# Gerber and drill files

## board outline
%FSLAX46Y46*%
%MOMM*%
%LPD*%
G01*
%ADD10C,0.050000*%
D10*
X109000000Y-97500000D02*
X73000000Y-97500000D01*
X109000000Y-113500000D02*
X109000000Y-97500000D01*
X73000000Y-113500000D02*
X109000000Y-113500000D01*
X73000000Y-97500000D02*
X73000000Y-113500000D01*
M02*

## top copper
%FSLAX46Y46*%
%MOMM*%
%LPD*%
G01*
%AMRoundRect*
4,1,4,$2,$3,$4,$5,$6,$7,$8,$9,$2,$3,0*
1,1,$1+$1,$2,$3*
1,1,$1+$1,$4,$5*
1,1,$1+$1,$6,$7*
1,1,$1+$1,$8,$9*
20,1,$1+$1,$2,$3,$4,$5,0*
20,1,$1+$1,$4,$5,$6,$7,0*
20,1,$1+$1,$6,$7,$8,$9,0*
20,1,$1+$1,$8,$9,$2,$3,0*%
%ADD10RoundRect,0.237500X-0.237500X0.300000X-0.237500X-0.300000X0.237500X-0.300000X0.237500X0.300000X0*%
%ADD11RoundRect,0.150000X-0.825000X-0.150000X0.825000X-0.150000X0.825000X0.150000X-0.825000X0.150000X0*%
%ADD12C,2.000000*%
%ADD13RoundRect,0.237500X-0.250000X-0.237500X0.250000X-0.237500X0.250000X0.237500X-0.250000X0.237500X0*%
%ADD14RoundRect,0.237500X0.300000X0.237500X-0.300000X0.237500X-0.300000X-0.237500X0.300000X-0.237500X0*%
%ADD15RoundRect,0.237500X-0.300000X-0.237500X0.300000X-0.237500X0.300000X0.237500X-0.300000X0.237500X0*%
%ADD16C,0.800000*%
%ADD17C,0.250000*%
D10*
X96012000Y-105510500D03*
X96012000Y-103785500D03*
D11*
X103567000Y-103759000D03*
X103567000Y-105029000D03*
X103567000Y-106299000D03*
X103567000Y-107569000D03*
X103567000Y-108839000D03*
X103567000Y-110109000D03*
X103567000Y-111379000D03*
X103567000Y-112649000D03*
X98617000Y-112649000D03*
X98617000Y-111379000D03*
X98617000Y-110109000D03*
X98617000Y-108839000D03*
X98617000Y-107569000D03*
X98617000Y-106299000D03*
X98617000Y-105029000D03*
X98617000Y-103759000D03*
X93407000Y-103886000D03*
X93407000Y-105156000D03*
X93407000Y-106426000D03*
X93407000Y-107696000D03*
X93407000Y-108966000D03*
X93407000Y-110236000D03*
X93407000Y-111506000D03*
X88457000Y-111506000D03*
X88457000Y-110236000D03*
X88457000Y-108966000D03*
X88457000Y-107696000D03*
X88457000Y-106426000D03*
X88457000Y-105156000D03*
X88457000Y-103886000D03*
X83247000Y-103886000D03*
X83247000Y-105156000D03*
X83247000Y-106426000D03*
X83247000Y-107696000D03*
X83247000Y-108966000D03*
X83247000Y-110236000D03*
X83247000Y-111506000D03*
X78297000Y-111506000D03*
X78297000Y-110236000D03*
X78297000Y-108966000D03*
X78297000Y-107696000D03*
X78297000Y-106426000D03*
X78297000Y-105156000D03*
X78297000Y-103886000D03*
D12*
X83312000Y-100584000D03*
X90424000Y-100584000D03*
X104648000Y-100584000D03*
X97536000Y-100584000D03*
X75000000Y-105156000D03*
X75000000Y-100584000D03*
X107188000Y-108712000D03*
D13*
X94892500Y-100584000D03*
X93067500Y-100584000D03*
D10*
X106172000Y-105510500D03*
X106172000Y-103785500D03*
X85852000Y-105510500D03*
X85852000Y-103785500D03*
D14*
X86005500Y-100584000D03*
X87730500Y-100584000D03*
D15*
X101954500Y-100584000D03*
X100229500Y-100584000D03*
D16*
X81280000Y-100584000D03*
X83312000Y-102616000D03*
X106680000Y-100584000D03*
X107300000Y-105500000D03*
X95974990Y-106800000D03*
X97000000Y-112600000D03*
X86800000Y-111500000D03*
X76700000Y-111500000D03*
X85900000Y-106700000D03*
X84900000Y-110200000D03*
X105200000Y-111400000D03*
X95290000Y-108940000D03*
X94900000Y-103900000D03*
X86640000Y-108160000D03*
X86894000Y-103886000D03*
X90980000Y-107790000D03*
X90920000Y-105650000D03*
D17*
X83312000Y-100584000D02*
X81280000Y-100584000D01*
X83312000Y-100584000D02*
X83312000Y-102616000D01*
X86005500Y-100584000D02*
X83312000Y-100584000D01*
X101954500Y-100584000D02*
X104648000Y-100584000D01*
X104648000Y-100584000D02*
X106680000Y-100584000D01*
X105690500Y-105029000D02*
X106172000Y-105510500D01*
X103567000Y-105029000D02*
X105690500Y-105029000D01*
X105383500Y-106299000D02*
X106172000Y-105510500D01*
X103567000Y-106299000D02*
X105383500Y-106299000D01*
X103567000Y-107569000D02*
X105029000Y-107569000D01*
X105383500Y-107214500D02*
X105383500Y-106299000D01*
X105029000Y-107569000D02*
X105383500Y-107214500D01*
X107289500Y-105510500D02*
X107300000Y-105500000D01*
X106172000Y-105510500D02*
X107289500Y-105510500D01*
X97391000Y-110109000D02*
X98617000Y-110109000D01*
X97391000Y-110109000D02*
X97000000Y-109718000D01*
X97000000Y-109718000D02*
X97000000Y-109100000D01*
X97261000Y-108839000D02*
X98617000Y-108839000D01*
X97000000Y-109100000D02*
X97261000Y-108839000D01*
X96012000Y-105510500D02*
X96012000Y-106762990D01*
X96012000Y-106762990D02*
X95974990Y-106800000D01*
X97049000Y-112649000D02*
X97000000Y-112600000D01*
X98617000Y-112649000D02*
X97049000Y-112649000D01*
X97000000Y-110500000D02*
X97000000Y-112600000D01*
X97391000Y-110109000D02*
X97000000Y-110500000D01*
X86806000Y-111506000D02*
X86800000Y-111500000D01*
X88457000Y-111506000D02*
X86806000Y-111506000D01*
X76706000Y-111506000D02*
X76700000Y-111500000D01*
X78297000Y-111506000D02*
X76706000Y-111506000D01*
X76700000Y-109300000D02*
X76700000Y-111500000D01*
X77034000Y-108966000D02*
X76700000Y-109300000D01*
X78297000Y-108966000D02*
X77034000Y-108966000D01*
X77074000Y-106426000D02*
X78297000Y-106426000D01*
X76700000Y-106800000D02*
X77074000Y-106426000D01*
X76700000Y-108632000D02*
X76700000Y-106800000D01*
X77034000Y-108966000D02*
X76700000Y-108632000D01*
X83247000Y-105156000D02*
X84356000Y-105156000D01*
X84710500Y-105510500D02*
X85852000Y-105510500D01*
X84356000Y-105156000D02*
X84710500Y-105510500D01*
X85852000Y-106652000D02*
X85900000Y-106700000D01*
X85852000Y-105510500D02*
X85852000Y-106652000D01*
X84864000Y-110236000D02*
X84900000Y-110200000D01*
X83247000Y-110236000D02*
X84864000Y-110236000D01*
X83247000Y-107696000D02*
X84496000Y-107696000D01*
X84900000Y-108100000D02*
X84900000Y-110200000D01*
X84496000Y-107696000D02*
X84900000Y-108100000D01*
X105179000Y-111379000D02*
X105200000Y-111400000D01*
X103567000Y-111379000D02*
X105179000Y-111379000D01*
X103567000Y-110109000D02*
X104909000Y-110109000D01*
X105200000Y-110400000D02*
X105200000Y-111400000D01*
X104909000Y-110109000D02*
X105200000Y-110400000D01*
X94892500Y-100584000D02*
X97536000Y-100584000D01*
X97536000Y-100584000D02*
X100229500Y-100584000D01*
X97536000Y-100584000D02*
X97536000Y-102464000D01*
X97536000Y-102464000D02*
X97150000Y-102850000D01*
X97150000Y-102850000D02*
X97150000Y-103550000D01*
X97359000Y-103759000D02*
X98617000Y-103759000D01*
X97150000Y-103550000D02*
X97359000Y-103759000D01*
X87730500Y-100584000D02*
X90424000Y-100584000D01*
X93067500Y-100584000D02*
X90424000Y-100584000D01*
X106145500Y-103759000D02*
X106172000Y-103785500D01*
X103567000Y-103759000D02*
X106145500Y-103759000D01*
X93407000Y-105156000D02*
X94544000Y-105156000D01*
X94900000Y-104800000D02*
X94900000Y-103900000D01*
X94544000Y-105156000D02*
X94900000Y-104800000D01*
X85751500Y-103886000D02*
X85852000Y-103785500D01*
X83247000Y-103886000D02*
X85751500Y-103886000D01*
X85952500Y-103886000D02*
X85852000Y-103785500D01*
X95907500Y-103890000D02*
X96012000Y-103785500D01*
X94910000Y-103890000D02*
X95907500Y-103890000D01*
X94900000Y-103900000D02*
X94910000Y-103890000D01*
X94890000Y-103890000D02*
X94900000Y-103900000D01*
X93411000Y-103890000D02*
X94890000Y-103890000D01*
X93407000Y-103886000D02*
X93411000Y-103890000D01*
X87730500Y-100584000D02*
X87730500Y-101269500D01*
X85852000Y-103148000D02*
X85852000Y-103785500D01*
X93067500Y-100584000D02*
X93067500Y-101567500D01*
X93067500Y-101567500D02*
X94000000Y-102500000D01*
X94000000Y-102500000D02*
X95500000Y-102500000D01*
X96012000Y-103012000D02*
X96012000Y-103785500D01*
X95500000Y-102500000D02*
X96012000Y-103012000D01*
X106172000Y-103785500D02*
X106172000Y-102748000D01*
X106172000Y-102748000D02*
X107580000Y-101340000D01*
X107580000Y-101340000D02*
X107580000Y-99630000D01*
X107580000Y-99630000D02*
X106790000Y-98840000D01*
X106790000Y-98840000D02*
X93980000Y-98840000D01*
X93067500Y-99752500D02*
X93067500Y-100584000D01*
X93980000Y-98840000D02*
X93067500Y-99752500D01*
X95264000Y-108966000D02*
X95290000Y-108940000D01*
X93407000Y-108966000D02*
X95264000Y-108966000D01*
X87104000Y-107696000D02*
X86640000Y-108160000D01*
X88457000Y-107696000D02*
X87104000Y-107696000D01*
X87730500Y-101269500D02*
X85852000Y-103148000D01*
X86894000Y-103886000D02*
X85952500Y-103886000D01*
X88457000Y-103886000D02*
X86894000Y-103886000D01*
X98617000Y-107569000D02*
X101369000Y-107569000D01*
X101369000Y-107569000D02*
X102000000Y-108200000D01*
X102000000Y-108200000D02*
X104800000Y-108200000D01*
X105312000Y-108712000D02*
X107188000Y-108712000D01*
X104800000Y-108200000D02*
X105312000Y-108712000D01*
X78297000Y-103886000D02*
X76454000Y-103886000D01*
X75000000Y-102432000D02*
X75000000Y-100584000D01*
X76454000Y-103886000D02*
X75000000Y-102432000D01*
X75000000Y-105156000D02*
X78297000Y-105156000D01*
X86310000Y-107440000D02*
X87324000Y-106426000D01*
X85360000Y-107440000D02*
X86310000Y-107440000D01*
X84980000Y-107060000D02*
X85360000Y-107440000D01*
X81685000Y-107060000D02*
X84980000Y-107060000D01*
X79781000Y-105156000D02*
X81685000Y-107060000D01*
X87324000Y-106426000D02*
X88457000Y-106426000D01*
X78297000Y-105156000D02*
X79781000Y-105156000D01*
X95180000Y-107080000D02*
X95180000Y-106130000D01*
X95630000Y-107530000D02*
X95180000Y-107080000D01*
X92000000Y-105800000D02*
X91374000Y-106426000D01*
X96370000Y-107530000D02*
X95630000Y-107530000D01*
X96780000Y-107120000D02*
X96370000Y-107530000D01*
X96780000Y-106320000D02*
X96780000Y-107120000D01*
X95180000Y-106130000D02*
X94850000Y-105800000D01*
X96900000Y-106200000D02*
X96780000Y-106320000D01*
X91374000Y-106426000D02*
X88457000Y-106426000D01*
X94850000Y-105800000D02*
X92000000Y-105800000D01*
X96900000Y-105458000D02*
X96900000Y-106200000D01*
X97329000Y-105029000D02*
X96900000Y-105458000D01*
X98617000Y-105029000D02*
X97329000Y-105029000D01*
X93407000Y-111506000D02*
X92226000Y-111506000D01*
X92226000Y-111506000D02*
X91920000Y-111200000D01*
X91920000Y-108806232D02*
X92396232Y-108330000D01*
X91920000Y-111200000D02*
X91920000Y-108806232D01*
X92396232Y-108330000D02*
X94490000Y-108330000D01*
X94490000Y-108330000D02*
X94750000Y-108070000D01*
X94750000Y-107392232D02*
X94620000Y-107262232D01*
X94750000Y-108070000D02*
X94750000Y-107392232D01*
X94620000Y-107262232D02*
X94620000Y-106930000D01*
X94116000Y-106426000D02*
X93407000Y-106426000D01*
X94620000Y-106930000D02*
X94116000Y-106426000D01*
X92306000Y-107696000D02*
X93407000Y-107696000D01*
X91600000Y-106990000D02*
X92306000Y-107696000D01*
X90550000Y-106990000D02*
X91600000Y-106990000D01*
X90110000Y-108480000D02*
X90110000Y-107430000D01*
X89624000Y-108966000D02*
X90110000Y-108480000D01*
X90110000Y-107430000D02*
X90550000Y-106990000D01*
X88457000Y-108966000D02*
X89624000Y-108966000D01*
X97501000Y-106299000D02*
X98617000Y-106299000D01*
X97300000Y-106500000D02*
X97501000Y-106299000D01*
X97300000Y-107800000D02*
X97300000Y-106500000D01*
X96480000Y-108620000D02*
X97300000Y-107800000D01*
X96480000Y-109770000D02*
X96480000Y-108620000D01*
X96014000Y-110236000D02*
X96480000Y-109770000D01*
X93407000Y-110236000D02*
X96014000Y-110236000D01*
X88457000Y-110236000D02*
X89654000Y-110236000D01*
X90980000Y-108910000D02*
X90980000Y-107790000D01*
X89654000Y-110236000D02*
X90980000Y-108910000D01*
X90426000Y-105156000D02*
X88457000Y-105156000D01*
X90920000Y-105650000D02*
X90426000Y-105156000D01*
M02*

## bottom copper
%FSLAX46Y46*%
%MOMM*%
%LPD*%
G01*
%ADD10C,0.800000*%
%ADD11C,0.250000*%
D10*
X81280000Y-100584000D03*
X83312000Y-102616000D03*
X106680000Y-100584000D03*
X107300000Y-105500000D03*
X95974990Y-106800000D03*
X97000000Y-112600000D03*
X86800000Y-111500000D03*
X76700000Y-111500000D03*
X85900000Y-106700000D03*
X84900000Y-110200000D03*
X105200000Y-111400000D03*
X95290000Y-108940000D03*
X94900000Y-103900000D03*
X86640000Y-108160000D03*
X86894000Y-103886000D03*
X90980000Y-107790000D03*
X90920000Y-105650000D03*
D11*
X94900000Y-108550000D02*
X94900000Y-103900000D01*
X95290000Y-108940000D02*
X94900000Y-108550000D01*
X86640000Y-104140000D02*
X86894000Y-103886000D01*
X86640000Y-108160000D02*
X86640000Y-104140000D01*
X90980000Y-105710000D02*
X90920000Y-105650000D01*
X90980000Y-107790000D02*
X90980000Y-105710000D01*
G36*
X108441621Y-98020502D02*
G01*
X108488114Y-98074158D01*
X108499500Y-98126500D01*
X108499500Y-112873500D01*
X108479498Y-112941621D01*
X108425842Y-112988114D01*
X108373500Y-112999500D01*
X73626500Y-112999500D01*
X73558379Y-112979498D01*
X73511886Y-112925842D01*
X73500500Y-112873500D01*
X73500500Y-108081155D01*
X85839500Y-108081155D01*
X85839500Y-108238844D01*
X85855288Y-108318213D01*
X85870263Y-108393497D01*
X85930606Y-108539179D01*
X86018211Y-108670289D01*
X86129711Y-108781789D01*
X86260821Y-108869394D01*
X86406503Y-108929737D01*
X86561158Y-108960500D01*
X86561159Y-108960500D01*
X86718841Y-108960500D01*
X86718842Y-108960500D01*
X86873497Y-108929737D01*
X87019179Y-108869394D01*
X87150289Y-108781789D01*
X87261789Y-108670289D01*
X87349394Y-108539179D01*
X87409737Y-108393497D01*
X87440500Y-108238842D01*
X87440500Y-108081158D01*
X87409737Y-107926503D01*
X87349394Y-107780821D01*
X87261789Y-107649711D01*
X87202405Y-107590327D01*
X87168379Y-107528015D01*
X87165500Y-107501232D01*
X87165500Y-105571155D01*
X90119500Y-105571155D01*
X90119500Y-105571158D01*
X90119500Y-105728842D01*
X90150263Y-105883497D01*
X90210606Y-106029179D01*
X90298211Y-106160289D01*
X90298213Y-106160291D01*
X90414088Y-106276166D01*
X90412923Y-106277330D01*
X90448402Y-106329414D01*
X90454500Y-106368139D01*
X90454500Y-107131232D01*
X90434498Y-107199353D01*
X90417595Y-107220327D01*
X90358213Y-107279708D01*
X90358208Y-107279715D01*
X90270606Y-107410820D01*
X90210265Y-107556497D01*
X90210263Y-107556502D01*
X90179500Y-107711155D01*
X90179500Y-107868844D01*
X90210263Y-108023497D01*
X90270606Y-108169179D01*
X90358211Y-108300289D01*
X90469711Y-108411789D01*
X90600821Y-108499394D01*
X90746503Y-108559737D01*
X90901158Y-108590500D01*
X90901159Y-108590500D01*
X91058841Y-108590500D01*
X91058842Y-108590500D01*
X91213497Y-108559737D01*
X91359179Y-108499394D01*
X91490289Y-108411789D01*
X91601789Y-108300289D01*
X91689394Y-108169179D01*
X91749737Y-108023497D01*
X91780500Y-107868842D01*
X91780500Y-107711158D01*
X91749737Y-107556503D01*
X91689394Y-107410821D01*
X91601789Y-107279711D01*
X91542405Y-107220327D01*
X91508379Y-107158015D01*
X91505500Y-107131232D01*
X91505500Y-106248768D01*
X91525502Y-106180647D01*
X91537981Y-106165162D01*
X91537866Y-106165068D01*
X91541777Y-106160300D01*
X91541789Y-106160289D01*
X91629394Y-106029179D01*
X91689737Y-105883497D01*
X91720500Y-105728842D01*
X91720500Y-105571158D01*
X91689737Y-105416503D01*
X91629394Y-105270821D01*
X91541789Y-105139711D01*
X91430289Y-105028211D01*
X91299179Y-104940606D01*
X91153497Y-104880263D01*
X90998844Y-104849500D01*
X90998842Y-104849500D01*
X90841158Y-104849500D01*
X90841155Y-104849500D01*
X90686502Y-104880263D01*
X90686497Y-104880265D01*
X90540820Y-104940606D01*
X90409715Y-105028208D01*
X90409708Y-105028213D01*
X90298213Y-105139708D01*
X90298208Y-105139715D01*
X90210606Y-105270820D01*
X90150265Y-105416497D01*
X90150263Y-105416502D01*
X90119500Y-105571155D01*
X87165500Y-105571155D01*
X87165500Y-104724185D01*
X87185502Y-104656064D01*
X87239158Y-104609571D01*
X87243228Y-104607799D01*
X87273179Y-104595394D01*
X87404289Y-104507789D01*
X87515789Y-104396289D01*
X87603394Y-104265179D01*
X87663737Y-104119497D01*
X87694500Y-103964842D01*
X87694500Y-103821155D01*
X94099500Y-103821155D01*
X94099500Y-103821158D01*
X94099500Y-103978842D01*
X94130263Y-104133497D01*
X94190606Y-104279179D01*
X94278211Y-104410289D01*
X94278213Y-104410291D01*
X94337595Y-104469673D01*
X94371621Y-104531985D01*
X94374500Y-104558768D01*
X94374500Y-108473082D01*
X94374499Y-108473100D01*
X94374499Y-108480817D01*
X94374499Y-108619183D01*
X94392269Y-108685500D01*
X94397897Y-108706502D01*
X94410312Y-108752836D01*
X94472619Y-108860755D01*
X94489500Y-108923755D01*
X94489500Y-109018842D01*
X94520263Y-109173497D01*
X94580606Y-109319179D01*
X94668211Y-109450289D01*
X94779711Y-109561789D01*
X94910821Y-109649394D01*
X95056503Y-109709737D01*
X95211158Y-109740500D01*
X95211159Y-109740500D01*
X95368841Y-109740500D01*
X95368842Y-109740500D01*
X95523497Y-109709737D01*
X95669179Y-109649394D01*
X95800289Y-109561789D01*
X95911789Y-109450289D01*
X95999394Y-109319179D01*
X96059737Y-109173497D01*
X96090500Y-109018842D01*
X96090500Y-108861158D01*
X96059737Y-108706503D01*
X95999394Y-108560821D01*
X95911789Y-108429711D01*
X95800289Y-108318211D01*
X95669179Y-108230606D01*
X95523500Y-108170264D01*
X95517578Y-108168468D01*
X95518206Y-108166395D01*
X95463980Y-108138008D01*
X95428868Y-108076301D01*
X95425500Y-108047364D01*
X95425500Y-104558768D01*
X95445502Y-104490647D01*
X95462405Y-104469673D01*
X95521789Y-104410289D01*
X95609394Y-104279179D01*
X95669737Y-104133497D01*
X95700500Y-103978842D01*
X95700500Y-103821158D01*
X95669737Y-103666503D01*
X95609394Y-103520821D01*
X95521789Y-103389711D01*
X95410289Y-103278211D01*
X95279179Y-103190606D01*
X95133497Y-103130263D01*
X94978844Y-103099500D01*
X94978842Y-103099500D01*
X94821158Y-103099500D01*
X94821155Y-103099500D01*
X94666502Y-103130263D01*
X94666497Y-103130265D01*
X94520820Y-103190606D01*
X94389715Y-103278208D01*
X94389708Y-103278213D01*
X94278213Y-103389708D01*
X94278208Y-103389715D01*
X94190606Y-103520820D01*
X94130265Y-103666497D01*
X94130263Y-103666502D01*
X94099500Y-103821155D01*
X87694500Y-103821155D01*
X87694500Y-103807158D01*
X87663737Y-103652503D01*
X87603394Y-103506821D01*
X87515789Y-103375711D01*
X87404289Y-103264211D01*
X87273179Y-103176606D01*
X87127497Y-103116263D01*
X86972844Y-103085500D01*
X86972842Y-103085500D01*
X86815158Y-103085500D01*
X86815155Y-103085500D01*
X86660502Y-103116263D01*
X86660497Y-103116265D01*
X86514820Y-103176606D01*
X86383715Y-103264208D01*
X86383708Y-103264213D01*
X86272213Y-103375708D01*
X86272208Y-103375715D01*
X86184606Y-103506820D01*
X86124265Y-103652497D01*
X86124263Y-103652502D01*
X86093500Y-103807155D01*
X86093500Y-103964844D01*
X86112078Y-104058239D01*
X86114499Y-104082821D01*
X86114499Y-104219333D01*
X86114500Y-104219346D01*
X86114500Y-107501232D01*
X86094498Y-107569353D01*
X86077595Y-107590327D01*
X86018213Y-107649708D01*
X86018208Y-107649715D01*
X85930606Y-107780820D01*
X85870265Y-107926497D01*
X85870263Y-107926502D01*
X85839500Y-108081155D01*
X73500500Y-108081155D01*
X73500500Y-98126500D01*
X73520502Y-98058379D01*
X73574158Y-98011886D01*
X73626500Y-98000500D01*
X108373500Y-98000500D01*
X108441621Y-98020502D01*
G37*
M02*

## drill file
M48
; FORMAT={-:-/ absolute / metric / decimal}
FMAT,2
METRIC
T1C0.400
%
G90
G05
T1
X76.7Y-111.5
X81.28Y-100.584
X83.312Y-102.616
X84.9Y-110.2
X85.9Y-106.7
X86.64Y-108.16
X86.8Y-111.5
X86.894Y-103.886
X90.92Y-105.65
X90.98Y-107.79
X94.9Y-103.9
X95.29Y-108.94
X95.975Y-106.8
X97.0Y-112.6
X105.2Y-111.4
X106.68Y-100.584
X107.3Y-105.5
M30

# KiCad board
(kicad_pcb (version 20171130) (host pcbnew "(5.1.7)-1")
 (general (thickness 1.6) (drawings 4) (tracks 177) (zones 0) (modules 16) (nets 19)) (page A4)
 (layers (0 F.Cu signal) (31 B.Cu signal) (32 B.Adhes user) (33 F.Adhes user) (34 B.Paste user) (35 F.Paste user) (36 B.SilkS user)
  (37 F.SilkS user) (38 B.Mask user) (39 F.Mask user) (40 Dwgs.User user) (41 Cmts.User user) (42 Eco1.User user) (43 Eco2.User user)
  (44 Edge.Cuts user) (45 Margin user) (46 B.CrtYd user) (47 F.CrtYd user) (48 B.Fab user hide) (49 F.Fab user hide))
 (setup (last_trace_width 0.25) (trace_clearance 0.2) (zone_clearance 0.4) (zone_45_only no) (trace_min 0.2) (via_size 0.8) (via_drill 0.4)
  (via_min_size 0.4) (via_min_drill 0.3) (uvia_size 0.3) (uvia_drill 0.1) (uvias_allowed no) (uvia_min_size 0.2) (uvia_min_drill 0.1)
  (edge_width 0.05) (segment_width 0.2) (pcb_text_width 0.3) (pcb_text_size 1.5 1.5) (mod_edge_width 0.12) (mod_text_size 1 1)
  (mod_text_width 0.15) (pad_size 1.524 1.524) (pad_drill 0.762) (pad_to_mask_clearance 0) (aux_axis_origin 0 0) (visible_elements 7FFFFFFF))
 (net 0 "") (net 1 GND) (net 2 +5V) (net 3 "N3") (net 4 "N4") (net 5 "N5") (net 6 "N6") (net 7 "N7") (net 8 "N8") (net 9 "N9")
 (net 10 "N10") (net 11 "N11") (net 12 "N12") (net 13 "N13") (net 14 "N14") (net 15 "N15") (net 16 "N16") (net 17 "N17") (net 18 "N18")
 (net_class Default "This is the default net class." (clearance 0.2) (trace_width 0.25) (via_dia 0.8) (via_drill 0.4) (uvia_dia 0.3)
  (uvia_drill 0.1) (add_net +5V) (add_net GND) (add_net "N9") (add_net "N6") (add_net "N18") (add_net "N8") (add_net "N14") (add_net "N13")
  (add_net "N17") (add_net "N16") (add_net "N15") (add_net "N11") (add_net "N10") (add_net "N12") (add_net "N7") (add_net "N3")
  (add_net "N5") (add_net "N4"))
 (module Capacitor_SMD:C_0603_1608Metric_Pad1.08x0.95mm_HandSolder (layer F.Cu) (at 96.012 104.648 270)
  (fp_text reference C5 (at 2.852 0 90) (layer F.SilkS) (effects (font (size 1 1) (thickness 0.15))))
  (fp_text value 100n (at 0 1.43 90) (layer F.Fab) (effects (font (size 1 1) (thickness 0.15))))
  (pad 2 smd roundrect (at 0.8625 0 270) (size 1.075 0.95) (layers F.Cu F.Paste F.Mask) (roundrect_rratio 0.25) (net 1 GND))
  (pad 1 smd roundrect (at -0.8625 0 270) (size 1.075 0.95) (layers F.Cu F.Paste F.Mask) (roundrect_rratio 0.25) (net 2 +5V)))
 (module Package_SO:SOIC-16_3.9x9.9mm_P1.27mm (layer F.Cu) (at 101.092 108.204)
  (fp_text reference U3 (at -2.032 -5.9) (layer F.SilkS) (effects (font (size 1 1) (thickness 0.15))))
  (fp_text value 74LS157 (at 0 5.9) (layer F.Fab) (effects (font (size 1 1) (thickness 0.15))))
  (pad 16 smd roundrect (at 2.475 -4.445) (size 1.95 0.6) (layers F.Cu F.Paste F.Mask) (roundrect_rratio 0.25) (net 2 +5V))
  (pad 15 smd roundrect (at 2.475 -3.175) (size 1.95 0.6) (layers F.Cu F.Paste F.Mask) (roundrect_rratio 0.25) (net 1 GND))
  (pad 14 smd roundrect (at 2.475 -1.905) (size 1.95 0.6) (layers F.Cu F.Paste F.Mask) (roundrect_rratio 0.25) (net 1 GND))
  (pad 13 smd roundrect (at 2.475 -0.635) (size 1.95 0.6) (layers F.Cu F.Paste F.Mask) (roundrect_rratio 0.25) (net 1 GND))
  (pad 12 smd roundrect (at 2.475 0.635) (size 1.95 0.6) (layers F.Cu F.Paste F.Mask) (roundrect_rratio 0.25) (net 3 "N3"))
  (pad 11 smd roundrect (at 2.475 1.905) (size 1.95 0.6) (layers F.Cu F.Paste F.Mask) (roundrect_rratio 0.25) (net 1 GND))
  (pad 10 smd roundrect (at 2.475 3.175) (size 1.95 0.6) (layers F.Cu F.Paste F.Mask) (roundrect_rratio 0.25) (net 1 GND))
  (pad 9 smd roundrect (at 2.475 4.445) (size 1.95 0.6) (layers F.Cu F.Paste F.Mask) (roundrect_rratio 0.25) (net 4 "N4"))
  (pad 8 smd roundrect (at -2.475 4.445) (size 1.95 0.6) (layers F.Cu F.Paste F.Mask) (roundrect_rratio 0.25) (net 1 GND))
  (pad 7 smd roundrect (at -2.475 3.175) (size 1.95 0.6) (layers F.Cu F.Paste F.Mask) (roundrect_rratio 0.25) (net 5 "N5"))
  (pad 6 smd roundrect (at -2.475 1.905) (size 1.95 0.6) (layers F.Cu F.Paste F.Mask) (roundrect_rratio 0.25) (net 1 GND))
  (pad 5 smd roundrect (at -2.475 0.635) (size 1.95 0.6) (layers F.Cu F.Paste F.Mask) (roundrect_rratio 0.25) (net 1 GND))
  (pad 4 smd roundrect (at -2.475 -0.635) (size 1.95 0.6) (layers F.Cu F.Paste F.Mask) (roundrect_rratio 0.25) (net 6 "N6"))
  (pad 3 smd roundrect (at -2.475 -1.905) (size 1.95 0.6) (layers F.Cu F.Paste F.Mask) (roundrect_rratio 0.25) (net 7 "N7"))
  (pad 2 smd roundrect (at -2.475 -3.175) (size 1.95 0.6) (layers F.Cu F.Paste F.Mask) (roundrect_rratio 0.25) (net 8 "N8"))
  (pad 1 smd roundrect (at -2.475 -4.445) (size 1.95 0.6) (layers F.Cu F.Paste F.Mask) (roundrect_rratio 0.25) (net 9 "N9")))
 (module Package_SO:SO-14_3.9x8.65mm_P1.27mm (layer F.Cu) (at 90.932 107.696)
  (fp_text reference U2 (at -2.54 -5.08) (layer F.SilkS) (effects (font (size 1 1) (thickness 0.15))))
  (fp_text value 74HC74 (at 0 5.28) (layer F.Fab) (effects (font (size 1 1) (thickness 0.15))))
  (pad 14 smd roundrect (at 2.475 -3.81) (size 1.95 0.6) (layers F.Cu F.Paste F.Mask) (roundrect_rratio 0.25) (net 2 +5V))
  (pad 13 smd roundrect (at 2.475 -2.54) (size 1.95 0.6) (layers F.Cu F.Paste F.Mask) (roundrect_rratio 0.25) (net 2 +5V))
  (pad 12 smd roundrect (at 2.475 -1.27) (size 1.95 0.6) (layers F.Cu F.Paste F.Mask) (roundrect_rratio 0.25) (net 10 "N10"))
  (pad 11 smd roundrect (at 2.475 0) (size 1.95 0.6) (layers F.Cu F.Paste F.Mask) (roundrect_rratio 0.25) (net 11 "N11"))
  (pad 10 smd roundrect (at 2.475 1.27) (size 1.95 0.6) (layers F.Cu F.Paste F.Mask) (roundrect_rratio 0.25) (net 2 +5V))
  (pad 9 smd roundrect (at 2.475 2.54) (size 1.95 0.6) (layers F.Cu F.Paste F.Mask) (roundrect_rratio 0.25) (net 7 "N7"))
  (pad 8 smd roundrect (at 2.475 3.81) (size 1.95 0.6) (layers F.Cu F.Paste F.Mask) (roundrect_rratio 0.25) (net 10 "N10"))
  (pad 7 smd roundrect (at -2.475 3.81) (size 1.95 0.6) (layers F.Cu F.Paste F.Mask) (roundrect_rratio 0.25) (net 1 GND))
  (pad 6 smd roundrect (at -2.475 2.54) (size 1.95 0.6) (layers F.Cu F.Paste F.Mask) (roundrect_rratio 0.25) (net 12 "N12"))
  (pad 5 smd roundrect (at -2.475 1.27) (size 1.95 0.6) (layers F.Cu F.Paste F.Mask) (roundrect_rratio 0.25) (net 11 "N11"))
  (pad 4 smd roundrect (at -2.475 0) (size 1.95 0.6) (layers F.Cu F.Paste F.Mask) (roundrect_rratio 0.25) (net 2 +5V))
  (pad 3 smd roundrect (at -2.475 -1.27) (size 1.95 0.6) (layers F.Cu F.Paste F.Mask) (roundrect_rratio 0.25) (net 8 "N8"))
  (pad 2 smd roundrect (at -2.475 -2.54) (size 1.95 0.6) (layers F.Cu F.Paste F.Mask) (roundrect_rratio 0.25) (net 12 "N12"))
  (pad 1 smd roundrect (at -2.475 -3.81) (size 1.95 0.6) (layers F.Cu F.Paste F.Mask) (roundrect_rratio 0.25) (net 2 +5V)))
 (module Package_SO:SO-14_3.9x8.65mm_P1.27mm (layer F.Cu) (at 80.772 107.696)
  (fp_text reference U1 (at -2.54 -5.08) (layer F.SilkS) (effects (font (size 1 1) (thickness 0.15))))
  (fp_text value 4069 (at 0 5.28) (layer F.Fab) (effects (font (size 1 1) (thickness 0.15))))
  (pad 14 smd roundrect (at 2.475 -3.81) (size 1.95 0.6) (layers F.Cu F.Paste F.Mask) (roundrect_rratio 0.25) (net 2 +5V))
  (pad 13 smd roundrect (at 2.475 -2.54) (size 1.95 0.6) (layers F.Cu F.Paste F.Mask) (roundrect_rratio 0.25) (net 1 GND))
  (pad 12 smd roundrect (at 2.475 -1.27) (size 1.95 0.6) (layers F.Cu F.Paste F.Mask) (roundrect_rratio 0.25) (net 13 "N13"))
  (pad 11 smd roundrect (at 2.475 0) (size 1.95 0.6) (layers F.Cu F.Paste F.Mask) (roundrect_rratio 0.25) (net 1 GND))
  (pad 10 smd roundrect (at 2.475 1.27) (size 1.95 0.6) (layers F.Cu F.Paste F.Mask) (roundrect_rratio 0.25) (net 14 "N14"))
  (pad 9 smd roundrect (at 2.475 2.54) (size 1.95 0.6) (layers F.Cu F.Paste F.Mask) (roundrect_rratio 0.25) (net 1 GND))
  (pad 8 smd roundrect (at 2.475 3.81) (size 1.95 0.6) (layers F.Cu F.Paste F.Mask) (roundrect_rratio 0.25) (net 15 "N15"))
  (pad 7 smd roundrect (at -2.475 3.81) (size 1.95 0.6) (layers F.Cu F.Paste F.Mask) (roundrect_rratio 0.25) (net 1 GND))
  (pad 6 smd roundrect (at -2.475 2.54) (size 1.95 0.6) (layers F.Cu F.Paste F.Mask) (roundrect_rratio 0.25) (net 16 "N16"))
  (pad 5 smd roundrect (at -2.475 1.27) (size 1.95 0.6) (layers F.Cu F.Paste F.Mask) (roundrect_rratio 0.25) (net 1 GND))
  (pad 4 smd roundrect (at -2.475 0) (size 1.95 0.6) (layers F.Cu F.Paste F.Mask) (roundrect_rratio 0.25) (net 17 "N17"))
  (pad 3 smd roundrect (at -2.475 -1.27) (size 1.95 0.6) (layers F.Cu F.Paste F.Mask) (roundrect_rratio 0.25) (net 1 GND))
  (pad 2 smd roundrect (at -2.475 -2.54) (size 1.95 0.6) (layers F.Cu F.Paste F.Mask) (roundrect_rratio 0.25) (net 8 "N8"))
  (pad 1 smd roundrect (at -2.475 -3.81) (size 1.95 0.6) (layers F.Cu F.Paste F.Mask) (roundrect_rratio 0.25) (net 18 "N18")))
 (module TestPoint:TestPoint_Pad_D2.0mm (layer F.Cu) (at 83.312 100.584 270)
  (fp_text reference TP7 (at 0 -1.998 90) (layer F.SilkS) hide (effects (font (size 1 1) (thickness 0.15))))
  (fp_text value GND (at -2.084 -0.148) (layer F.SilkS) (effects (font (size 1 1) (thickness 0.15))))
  (pad 1 smd circle (at 0 0 270) (size 2 2) (layers F.Cu F.Mask) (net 1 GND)))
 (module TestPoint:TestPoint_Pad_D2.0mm (layer F.Cu) (at 90.424 100.584 270)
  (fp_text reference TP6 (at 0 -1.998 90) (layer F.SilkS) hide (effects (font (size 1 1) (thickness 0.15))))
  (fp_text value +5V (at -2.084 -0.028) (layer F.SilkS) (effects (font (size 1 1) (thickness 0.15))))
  (pad 1 smd circle (at 0 0 270) (size 2 2) (layers F.Cu F.Mask) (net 2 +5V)))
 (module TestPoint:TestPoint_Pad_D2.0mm (layer F.Cu) (at 104.648 100.584)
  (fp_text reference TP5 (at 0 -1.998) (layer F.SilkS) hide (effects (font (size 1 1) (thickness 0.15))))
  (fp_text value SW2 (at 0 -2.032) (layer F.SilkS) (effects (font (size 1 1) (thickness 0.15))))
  (pad 1 smd circle (at 0 0) (size 2 2) (layers F.Cu F.Mask) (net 1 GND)))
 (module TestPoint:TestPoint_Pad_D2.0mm (layer F.Cu) (at 97.536 100.584)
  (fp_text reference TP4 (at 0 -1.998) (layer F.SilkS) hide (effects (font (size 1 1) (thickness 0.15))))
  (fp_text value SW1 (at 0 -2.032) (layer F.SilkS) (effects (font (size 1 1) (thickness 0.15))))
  (pad 1 smd circle (at 0 0) (size 2 2) (layers F.Cu F.Mask) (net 9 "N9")))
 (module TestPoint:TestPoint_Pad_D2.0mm (layer F.Cu) (at 75 105.156)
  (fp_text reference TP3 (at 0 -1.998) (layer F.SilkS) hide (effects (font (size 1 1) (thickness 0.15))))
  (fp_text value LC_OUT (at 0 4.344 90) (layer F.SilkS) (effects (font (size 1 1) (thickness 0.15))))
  (pad 1 smd circle (at 0 0) (size 2 2) (layers F.Cu F.Mask) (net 8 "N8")))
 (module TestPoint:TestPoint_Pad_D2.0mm (layer F.Cu) (at 75 100.584)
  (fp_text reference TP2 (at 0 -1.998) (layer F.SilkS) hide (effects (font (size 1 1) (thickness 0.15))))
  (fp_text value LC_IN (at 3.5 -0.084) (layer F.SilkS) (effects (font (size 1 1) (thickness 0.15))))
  (pad 1 smd circle (at 0 0) (size 2 2) (layers F.Cu F.Mask) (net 18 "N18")))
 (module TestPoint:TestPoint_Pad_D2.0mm (layer F.Cu) (at 107.188 108.712)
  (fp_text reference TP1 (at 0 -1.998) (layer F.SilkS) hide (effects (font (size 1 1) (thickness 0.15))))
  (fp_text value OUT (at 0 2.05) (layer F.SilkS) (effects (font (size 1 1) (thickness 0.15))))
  (pad 1 smd circle (at 0 0) (size 2 2) (layers F.Cu F.Mask) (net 6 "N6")))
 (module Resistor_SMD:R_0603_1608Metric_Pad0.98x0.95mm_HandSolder (layer F.Cu) (at 93.98 100.584)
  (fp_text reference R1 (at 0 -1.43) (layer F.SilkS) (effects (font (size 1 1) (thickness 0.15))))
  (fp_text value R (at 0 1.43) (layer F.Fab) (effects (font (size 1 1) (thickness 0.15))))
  (pad 2 smd roundrect (at 0.9125 0) (size 0.975 0.95) (layers F.Cu F.Paste F.Mask) (roundrect_rratio 0.25) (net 9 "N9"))
  (pad 1 smd roundrect (at -0.9125 0) (size 0.975 0.95) (layers F.Cu F.Paste F.Mask) (roundrect_rratio 0.25) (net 2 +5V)))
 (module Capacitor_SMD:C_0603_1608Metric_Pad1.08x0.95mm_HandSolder (layer F.Cu) (at 106.172 104.648 270)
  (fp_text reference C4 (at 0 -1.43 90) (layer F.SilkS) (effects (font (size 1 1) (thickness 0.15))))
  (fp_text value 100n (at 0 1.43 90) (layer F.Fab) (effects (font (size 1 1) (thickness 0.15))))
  (pad 2 smd roundrect (at 0.8625 0 270) (size 1.075 0.95) (layers F.Cu F.Paste F.Mask) (roundrect_rratio 0.25) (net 1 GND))
  (pad 1 smd roundrect (at -0.8625 0 270) (size 1.075 0.95) (layers F.Cu F.Paste F.Mask) (roundrect_rratio 0.25) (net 2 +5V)))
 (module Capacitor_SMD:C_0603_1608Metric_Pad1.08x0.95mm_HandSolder (layer F.Cu) (at 85.852 104.648 270)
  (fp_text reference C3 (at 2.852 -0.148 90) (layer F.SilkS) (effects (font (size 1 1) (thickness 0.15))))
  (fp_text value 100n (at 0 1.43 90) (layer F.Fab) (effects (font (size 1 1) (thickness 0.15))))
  (pad 2 smd roundrect (at 0.8625 0 270) (size 1.075 0.95) (layers F.Cu F.Paste F.Mask) (roundrect_rratio 0.25) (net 1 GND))
  (pad 1 smd roundrect (at -0.8625 0 270) (size 1.075 0.95) (layers F.Cu F.Paste F.Mask) (roundrect_rratio 0.25) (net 2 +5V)))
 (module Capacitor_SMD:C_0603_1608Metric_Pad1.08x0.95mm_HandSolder (layer F.Cu) (at 86.868 100.584 180)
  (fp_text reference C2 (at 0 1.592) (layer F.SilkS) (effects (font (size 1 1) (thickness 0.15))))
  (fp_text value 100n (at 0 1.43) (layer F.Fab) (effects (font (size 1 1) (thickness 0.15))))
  (pad 2 smd roundrect (at 0.8625 0 180) (size 1.075 0.95) (layers F.Cu F.Paste F.Mask) (roundrect_rratio 0.25) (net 1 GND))
  (pad 1 smd roundrect (at -0.8625 0 180) (size 1.075 0.95) (layers F.Cu F.Paste F.Mask) (roundrect_rratio 0.25) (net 2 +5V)))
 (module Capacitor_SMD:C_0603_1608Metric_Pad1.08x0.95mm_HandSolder (layer F.Cu) (at 101.092 100.584)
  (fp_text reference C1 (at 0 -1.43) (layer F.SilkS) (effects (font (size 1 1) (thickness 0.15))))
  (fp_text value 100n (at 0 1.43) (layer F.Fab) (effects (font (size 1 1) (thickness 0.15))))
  (pad 2 smd roundrect (at 0.8625 0) (size 1.075 0.95) (layers F.Cu F.Paste F.Mask) (roundrect_rratio 0.25) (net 1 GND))
  (pad 1 smd roundrect (at -0.8625 0) (size 1.075 0.95) (layers F.Cu F.Paste F.Mask) (roundrect_rratio 0.25) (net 9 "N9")))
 (gr_line (start 109 97.5) (end 73 97.5) (layer Edge.Cuts) (width 0.05))
 (gr_line (start 109 113.5) (end 109 97.5) (layer Edge.Cuts) (width 0.05))
 (gr_line (start 73 113.5) (end 109 113.5) (layer Edge.Cuts) (width 0.05))
 (gr_line (start 73 97.5) (end 73 113.5) (layer Edge.Cuts) (width 0.05))
 (via (at 81.28 100.584) (size 0.8) (drill 0.4) (layers F.Cu B.Cu) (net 1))
 (segment (start 83.312 100.584) (end 81.28 100.584) (width 0.25) (layer F.Cu) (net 1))
 (via (at 83.312 102.616) (size 0.8) (drill 0.4) (layers F.Cu B.Cu) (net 1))
 (segment (start 83.312 100.584) (end 83.312 102.616) (width 0.25) (layer F.Cu) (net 1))
 (segment (start 86.0055 100.584) (end 83.312 100.584) (width 0.25) (layer F.Cu) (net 1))
 (segment (start 101.9545 100.584) (end 104.648 100.584) (width 0.25) (layer F.Cu) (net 1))
 (via (at 106.68 100.584) (size 0.8) (drill 0.4) (layers F.Cu B.Cu) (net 1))
 (segment (start 104.648 100.584) (end 106.68 100.584) (width 0.25) (layer F.Cu) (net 1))
 (segment (start 105.6905 105.029) (end 106.172 105.5105) (width 0.25) (layer F.Cu) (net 1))
 (segment (start 103.567 105.029) (end 105.6905 105.029) (width 0.25) (layer F.Cu) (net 1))
 (segment (start 105.3835 106.299) (end 106.172 105.5105) (width 0.25) (layer F.Cu) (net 1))
 (segment (start 103.567 106.299) (end 105.3835 106.299) (width 0.25) (layer F.Cu) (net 1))
 (segment (start 103.567 107.569) (end 105.029 107.569) (width 0.25) (layer F.Cu) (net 1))
 (segment (start 105.3835 107.2145) (end 105.3835 106.299) (width 0.25) (layer F.Cu) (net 1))
 (segment (start 105.029 107.569) (end 105.3835 107.2145) (width 0.25) (layer F.Cu) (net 1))
 (via (at 107.3 105.5) (size 0.8) (drill 0.4) (layers F.Cu B.Cu) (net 1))
 (segment (start 107.2895 105.5105) (end 107.3 105.5) (width 0.25) (layer F.Cu) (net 1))
 (segment (start 106.172 105.5105) (end 107.2895 105.5105) (width 0.25) (layer F.Cu) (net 1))
 (segment (start 97.391 110.109) (end 98.617 110.109) (width 0.25) (layer F.Cu) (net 1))
 (segment (start 97.391 110.109) (end 97 109.718) (width 0.25) (layer F.Cu) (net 1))
 (segment (start 97 109.718) (end 97 109.1) (width 0.25) (layer F.Cu) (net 1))
 (segment (start 97.261 108.839) (end 98.617 108.839) (width 0.25) (layer F.Cu) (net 1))
 (segment (start 97 109.1) (end 97.261 108.839) (width 0.25) (layer F.Cu) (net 1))
 (segment (start 96.012 105.5105) (end 96.012 106.76299) (width 0.25) (layer F.Cu) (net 1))
 (via (at 95.97499 106.8) (size 0.8) (drill 0.4) (layers F.Cu B.Cu) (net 1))
 (segment (start 96.012 106.76299) (end 95.97499 106.8) (width 0.25) (layer F.Cu) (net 1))
 (via (at 97 112.6) (size 0.8) (drill 0.4) (layers F.Cu B.Cu) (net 1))
 (segment (start 97.049 112.649) (end 97 112.6) (width 0.25) (layer F.Cu) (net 1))
 (segment (start 98.617 112.649) (end 97.049 112.649) (width 0.25) (layer F.Cu) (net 1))
 (segment (start 97 110.5) (end 97 112.6) (width 0.25) (layer F.Cu) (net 1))
 (segment (start 97.391 110.109) (end 97 110.5) (width 0.25) (layer F.Cu) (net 1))
 (via (at 86.8 111.5) (size 0.8) (drill 0.4) (layers F.Cu B.Cu) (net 1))
 (segment (start 86.806 111.506) (end 86.8 111.5) (width 0.25) (layer F.Cu) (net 1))
 (segment (start 88.457 111.506) (end 86.806 111.506) (width 0.25) (layer F.Cu) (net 1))
 (via (at 76.7 111.5) (size 0.8) (drill 0.4) (layers F.Cu B.Cu) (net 1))
 (segment (start 76.706 111.506) (end 76.7 111.5) (width 0.25) (layer F.Cu) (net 1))
 (segment (start 78.297 111.506) (end 76.706 111.506) (width 0.25) (layer F.Cu) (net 1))
 (segment (start 76.7 109.3) (end 76.7 111.5) (width 0.25) (layer F.Cu) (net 1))
 (segment (start 77.034 108.966) (end 76.7 109.3) (width 0.25) (layer F.Cu) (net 1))
 (segment (start 78.297 108.966) (end 77.034 108.966) (width 0.25) (layer F.Cu) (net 1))
 (segment (start 77.074 106.426) (end 78.297 106.426) (width 0.25) (layer F.Cu) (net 1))
 (segment (start 76.7 106.8) (end 77.074 106.426) (width 0.25) (layer F.Cu) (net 1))
 (segment (start 76.7 108.632) (end 76.7 106.8) (width 0.25) (layer F.Cu) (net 1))
 (segment (start 77.034 108.966) (end 76.7 108.632) (width 0.25) (layer F.Cu) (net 1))
 (segment (start 83.247 105.156) (end 84.356 105.156) (width 0.25) (layer F.Cu) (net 1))
 (segment (start 84.7105 105.5105) (end 85.852 105.5105) (width 0.25) (layer F.Cu) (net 1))
 (segment (start 84.356 105.156) (end 84.7105 105.5105) (width 0.25) (layer F.Cu) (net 1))
 (via (at 85.9 106.7) (size 0.8) (drill 0.4) (layers F.Cu B.Cu) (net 1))
 (segment (start 85.852 106.652) (end 85.9 106.7) (width 0.25) (layer F.Cu) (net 1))
 (segment (start 85.852 105.5105) (end 85.852 106.652) (width 0.25) (layer F.Cu) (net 1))
 (via (at 84.9 110.2) (size 0.8) (drill 0.4) (layers F.Cu B.Cu) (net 1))
 (segment (start 84.864 110.236) (end 84.9 110.2) (width 0.25) (layer F.Cu) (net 1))
 (segment (start 83.247 110.236) (end 84.864 110.236) (width 0.25) (layer F.Cu) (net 1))
 (segment (start 83.247 107.696) (end 84.496 107.696) (width 0.25) (layer F.Cu) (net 1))
 (segment (start 84.9 108.1) (end 84.9 110.2) (width 0.25) (layer F.Cu) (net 1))
 (segment (start 84.496 107.696) (end 84.9 108.1) (width 0.25) (layer F.Cu) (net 1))
 (via (at 105.2 111.4) (size 0.8) (drill 0.4) (layers F.Cu B.Cu) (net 1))
 (segment (start 105.179 111.379) (end 105.2 111.4) (width 0.25) (layer F.Cu) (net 1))
 (segment (start 103.567 111.379) (end 105.179 111.379) (width 0.25) (layer F.Cu) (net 1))
 (segment (start 103.567 110.109) (end 104.909 110.109) (width 0.25) (layer F.Cu) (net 1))
 (segment (start 105.2 110.4) (end 105.2 111.4) (width 0.25) (layer F.Cu) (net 1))
 (segment (start 104.909 110.109) (end 105.2 110.4) (width 0.25) (layer F.Cu) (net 1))
 (segment (start 94.8925 100.584) (end 97.536 100.584) (width 0.25) (layer F.Cu) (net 9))
 (segment (start 97.536 100.584) (end 100.2295 100.584) (width 0.25) (layer F.Cu) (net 9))
 (segment (start 97.536 100.584) (end 97.536 102.464) (width 0.25) (layer F.Cu) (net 9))
 (segment (start 97.536 102.464) (end 97.15 102.85) (width 0.25) (layer F.Cu) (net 9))
 (segment (start 97.15 102.85) (end 97.15 103.55) (width 0.25) (layer F.Cu) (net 9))
 (segment (start 97.359 103.759) (end 98.617 103.759) (width 0.25) (layer F.Cu) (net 9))
 (segment (start 97.15 103.55) (end 97.359 103.759) (width 0.25) (layer F.Cu) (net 9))
 (segment (start 87.7305 100.584) (end 90.424 100.584) (width 0.25) (layer F.Cu) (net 2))
 (segment (start 93.0675 100.584) (end 90.424 100.584) (width 0.25) (layer F.Cu) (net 2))
 (segment (start 106.1455 103.759) (end 106.172 103.7855) (width 0.25) (layer F.Cu) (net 2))
 (segment (start 103.567 103.759) (end 106.1455 103.759) (width 0.25) (layer F.Cu) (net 2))
 (segment (start 93.407 105.156) (end 94.544 105.156) (width 0.25) (layer F.Cu) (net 2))
 (segment (start 94.9 104.8) (end 94.9 103.9) (width 0.25) (layer F.Cu) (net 2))
 (segment (start 94.544 105.156) (end 94.9 104.8) (width 0.25) (layer F.Cu) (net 2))
 (segment (start 85.7515 103.886) (end 85.852 103.7855) (width 0.25) (layer F.Cu) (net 2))
 (segment (start 83.247 103.886) (end 85.7515 103.886) (width 0.25) (layer F.Cu) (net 2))
 (segment (start 85.9525 103.886) (end 85.852 103.7855) (width 0.25) (layer F.Cu) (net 2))
 (segment (start 95.9075 103.89) (end 96.012 103.7855) (width 0.25) (layer F.Cu) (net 2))
 (segment (start 94.91 103.89) (end 95.9075 103.89) (width 0.25) (layer F.Cu) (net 2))
 (segment (start 94.9 103.9) (end 94.91 103.89) (width 0.25) (layer F.Cu) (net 2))
 (segment (start 94.89 103.89) (end 94.9 103.9) (width 0.25) (layer F.Cu) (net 2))
 (segment (start 93.411 103.89) (end 94.89 103.89) (width 0.25) (layer F.Cu) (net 2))
 (segment (start 93.407 103.886) (end 93.411 103.89) (width 0.25) (layer F.Cu) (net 2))
 (segment (start 87.7305 100.584) (end 87.7305 101.2695) (width 0.25) (layer F.Cu) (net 2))
 (segment (start 85.852 103.148) (end 85.852 103.7855) (width 0.25) (layer F.Cu) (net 2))
 (segment (start 93.0675 100.584) (end 93.0675 101.5675) (width 0.25) (layer F.Cu) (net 2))
 (segment (start 93.0675 101.5675) (end 94 102.5) (width 0.25) (layer F.Cu) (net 2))
 (segment (start 94 102.5) (end 95.5 102.5) (width 0.25) (layer F.Cu) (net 2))
 (segment (start 96.012 103.012) (end 96.012 103.7855) (width 0.25) (layer F.Cu) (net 2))
 (segment (start 95.5 102.5) (end 96.012 103.012) (width 0.25) (layer F.Cu) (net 2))
 (segment (start 106.172 103.7855) (end 106.172 102.748) (width 0.25) (layer F.Cu) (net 2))
 (segment (start 106.172 102.748) (end 107.58 101.34) (width 0.25) (layer F.Cu) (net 2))
 (segment (start 107.58 101.34) (end 107.58 99.63) (width 0.25) (layer F.Cu) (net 2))
 (segment (start 107.58 99.63) (end 106.79 98.84) (width 0.25) (layer F.Cu) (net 2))
 (segment (start 106.79 98.84) (end 93.98 98.84) (width 0.25) (layer F.Cu) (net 2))
 (segment (start 93.0675 99.7525) (end 93.0675 100.584) (width 0.25) (layer F.Cu) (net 2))
 (segment (start 93.98 98.84) (end 93.0675 99.7525) (width 0.25) (layer F.Cu) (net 2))
 (via (at 95.29 108.94) (size 0.8) (drill 0.4) (layers F.Cu B.Cu) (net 2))
 (segment (start 95.264 108.966) (end 95.29 108.94) (width 0.25) (layer F.Cu) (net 2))
 (segment (start 93.407 108.966) (end 95.264 108.966) (width 0.25) (layer F.Cu) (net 2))
 (via (at 94.9 103.9) (size 0.8) (drill 0.4) (layers F.Cu B.Cu) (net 2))
 (segment (start 94.9 108.55) (end 94.9 103.9) (width 0.25) (layer B.Cu) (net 2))
 (segment (start 95.29 108.94) (end 94.9 108.55) (width 0.25) (layer B.Cu) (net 2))
 (segment (start 87.104 107.696) (end 86.64 108.16) (width 0.25) (layer F.Cu) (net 2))
 (via (at 86.64 108.16) (size 0.8) (drill 0.4) (layers F.Cu B.Cu) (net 2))
 (segment (start 88.457 107.696) (end 87.104 107.696) (width 0.25) (layer F.Cu) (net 2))
 (segment (start 87.7305 101.2695) (end 85.852 103.148) (width 0.25) (layer F.Cu) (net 2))
 (via (at 86.894 103.886) (size 0.8) (drill 0.4) (layers F.Cu B.Cu) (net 2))
 (segment (start 86.64 104.14) (end 86.894 103.886) (width 0.25) (layer B.Cu) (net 2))
 (segment (start 86.64 108.16) (end 86.64 104.14) (width 0.25) (layer B.Cu) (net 2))
 (segment (start 86.894 103.886) (end 85.9525 103.886) (width 0.25) (layer F.Cu) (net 2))
 (segment (start 88.457 103.886) (end 86.894 103.886) (width 0.25) (layer F.Cu) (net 2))
 (segment (start 98.617 107.569) (end 101.369 107.569) (width 0.25) (layer F.Cu) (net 6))
 (segment (start 101.369 107.569) (end 102 108.2) (width 0.25) (layer F.Cu) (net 6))
 (segment (start 102 108.2) (end 104.8 108.2) (width 0.25) (layer F.Cu) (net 6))
 (segment (start 105.312 108.712) (end 107.188 108.712) (width 0.25) (layer F.Cu) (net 6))
 (segment (start 104.8 108.2) (end 105.312 108.712) (width 0.25) (layer F.Cu) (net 6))
 (segment (start 78.297 103.886) (end 76.454 103.886) (width 0.25) (layer F.Cu) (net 18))
 (segment (start 75 102.432) (end 75 100.584) (width 0.25) (layer F.Cu) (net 18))
 (segment (start 76.454 103.886) (end 75 102.432) (width 0.25) (layer F.Cu) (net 18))
 (segment (start 75 105.156) (end 78.297 105.156) (width 0.25) (layer F.Cu) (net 8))
 (segment (start 86.31 107.44) (end 87.324 106.426) (width 0.25) (layer F.Cu) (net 8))
 (segment (start 85.36 107.44) (end 86.31 107.44) (width 0.25) (layer F.Cu) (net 8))
 (segment (start 84.98 107.06) (end 85.36 107.44) (width 0.25) (layer F.Cu) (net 8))
 (segment (start 81.685 107.06) (end 84.98 107.06) (width 0.25) (layer F.Cu) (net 8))
 (segment (start 79.781 105.156) (end 81.685 107.06) (width 0.25) (layer F.Cu) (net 8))
 (segment (start 87.324 106.426) (end 88.457 106.426) (width 0.25) (layer F.Cu) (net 8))
 (segment (start 78.297 105.156) (end 79.781 105.156) (width 0.25) (layer F.Cu) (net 8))
 (segment (start 95.18 107.08) (end 95.18 106.13) (width 0.25) (layer F.Cu) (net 8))
 (segment (start 95.63 107.53) (end 95.18 107.08) (width 0.25) (layer F.Cu) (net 8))
 (segment (start 92 105.8) (end 91.374 106.426) (width 0.25) (layer F.Cu) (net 8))
 (segment (start 96.37 107.53) (end 95.63 107.53) (width 0.25) (layer F.Cu) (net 8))
 (segment (start 96.78 107.12) (end 96.37 107.53) (width 0.25) (layer F.Cu) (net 8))
 (segment (start 96.78 106.32) (end 96.78 107.12) (width 0.25) (layer F.Cu) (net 8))
 (segment (start 95.18 106.13) (end 94.85 105.8) (width 0.25) (layer F.Cu) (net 8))
 (segment (start 96.9 106.2) (end 96.78 106.32) (width 0.25) (layer F.Cu) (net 8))
 (segment (start 91.374 106.426) (end 88.457 106.426) (width 0.25) (layer F.Cu) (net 8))
 (segment (start 94.85 105.8) (end 92 105.8) (width 0.25) (layer F.Cu) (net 8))
 (segment (start 96.9 105.458) (end 96.9 106.2) (width 0.25) (layer F.Cu) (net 8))
 (segment (start 97.329 105.029) (end 96.9 105.458) (width 0.25) (layer F.Cu) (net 8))
 (segment (start 98.617 105.029) (end 97.329 105.029) (width 0.25) (layer F.Cu) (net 8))
 (segment (start 93.407 111.506) (end 92.226 111.506) (width 0.25) (layer F.Cu) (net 10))
 (segment (start 92.226 111.506) (end 91.92 111.2) (width 0.25) (layer F.Cu) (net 10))
 (segment (start 91.92 108.806232) (end 92.396232 108.33) (width 0.25) (layer F.Cu) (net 10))
 (segment (start 91.92 111.2) (end 91.92 108.806232) (width 0.25) (layer F.Cu) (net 10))
 (segment (start 92.396232 108.33) (end 94.49 108.33) (width 0.25) (layer F.Cu) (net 10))
 (segment (start 94.49 108.33) (end 94.75 108.07) (width 0.25) (layer F.Cu) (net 10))
 (segment (start 94.75 107.392232) (end 94.62 107.262232) (width 0.25) (layer F.Cu) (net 10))
 (segment (start 94.75 108.07) (end 94.75 107.392232) (width 0.25) (layer F.Cu) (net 10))
 (segment (start 94.62 107.262232) (end 94.62 106.93) (width 0.25) (layer F.Cu) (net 10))
 (segment (start 94.116 106.426) (end 93.407 106.426) (width 0.25) (layer F.Cu) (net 10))
 (segment (start 94.62 106.93) (end 94.116 106.426) (width 0.25) (layer F.Cu) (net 10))
 (segment (start 92.306 107.696) (end 93.407 107.696) (width 0.25) (layer F.Cu) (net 11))
 (segment (start 91.6 106.99) (end 92.306 107.696) (width 0.25) (layer F.Cu) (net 11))
 (segment (start 90.55 106.99) (end 91.6 106.99) (width 0.25) (layer F.Cu) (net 11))
 (segment (start 90.11 108.48) (end 90.11 107.43) (width 0.25) (layer F.Cu) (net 11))
 (segment (start 89.624 108.966) (end 90.11 108.48) (width 0.25) (layer F.Cu) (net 11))
 (segment (start 90.11 107.43) (end 90.55 106.99) (width 0.25) (layer F.Cu) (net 11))
 (segment (start 88.457 108.966) (end 89.624 108.966) (width 0.25) (layer F.Cu) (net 11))
 (segment (start 97.501 106.299) (end 98.617 106.299) (width 0.25) (layer F.Cu) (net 7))
 (segment (start 97.3 106.5) (end 97.501 106.299) (width 0.25) (layer F.Cu) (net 7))
 (segment (start 97.3 107.8) (end 97.3 106.5) (width 0.25) (layer F.Cu) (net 7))
 (segment (start 96.48 108.62) (end 97.3 107.8) (width 0.25) (layer F.Cu) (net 7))
 (segment (start 96.48 109.77) (end 96.48 108.62) (width 0.25) (layer F.Cu) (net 7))
 (segment (start 96.014 110.236) (end 96.48 109.77) (width 0.25) (layer F.Cu) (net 7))
 (segment (start 93.407 110.236) (end 96.014 110.236) (width 0.25) (layer F.Cu) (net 7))
 (segment (start 88.457 110.236) (end 89.654 110.236) (width 0.25) (layer F.Cu) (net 12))
 (via (at 90.98 107.79) (size 0.8) (drill 0.4) (layers F.Cu B.Cu) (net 12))
 (segment (start 90.98 108.91) (end 90.98 107.79) (width 0.25) (layer F.Cu) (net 12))
 (segment (start 89.654 110.236) (end 90.98 108.91) (width 0.25) (layer F.Cu) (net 12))
 (via (at 90.92 105.65) (size 0.8) (drill 0.4) (layers F.Cu B.Cu) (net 12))
 (segment (start 90.98 105.71) (end 90.92 105.65) (width 0.25) (layer B.Cu) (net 12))
 (segment (start 90.98 107.79) (end 90.98 105.71) (width 0.25) (layer B.Cu) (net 12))
 (segment (start 90.426 105.156) (end 88.457 105.156) (width 0.25) (layer F.Cu) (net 12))
 (segment (start 90.92 105.65) (end 90.426 105.156) (width 0.25) (layer F.Cu) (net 12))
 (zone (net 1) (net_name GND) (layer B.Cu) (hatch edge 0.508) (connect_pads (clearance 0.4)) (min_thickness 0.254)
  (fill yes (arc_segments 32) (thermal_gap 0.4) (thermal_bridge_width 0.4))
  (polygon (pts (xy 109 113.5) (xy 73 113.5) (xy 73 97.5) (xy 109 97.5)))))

